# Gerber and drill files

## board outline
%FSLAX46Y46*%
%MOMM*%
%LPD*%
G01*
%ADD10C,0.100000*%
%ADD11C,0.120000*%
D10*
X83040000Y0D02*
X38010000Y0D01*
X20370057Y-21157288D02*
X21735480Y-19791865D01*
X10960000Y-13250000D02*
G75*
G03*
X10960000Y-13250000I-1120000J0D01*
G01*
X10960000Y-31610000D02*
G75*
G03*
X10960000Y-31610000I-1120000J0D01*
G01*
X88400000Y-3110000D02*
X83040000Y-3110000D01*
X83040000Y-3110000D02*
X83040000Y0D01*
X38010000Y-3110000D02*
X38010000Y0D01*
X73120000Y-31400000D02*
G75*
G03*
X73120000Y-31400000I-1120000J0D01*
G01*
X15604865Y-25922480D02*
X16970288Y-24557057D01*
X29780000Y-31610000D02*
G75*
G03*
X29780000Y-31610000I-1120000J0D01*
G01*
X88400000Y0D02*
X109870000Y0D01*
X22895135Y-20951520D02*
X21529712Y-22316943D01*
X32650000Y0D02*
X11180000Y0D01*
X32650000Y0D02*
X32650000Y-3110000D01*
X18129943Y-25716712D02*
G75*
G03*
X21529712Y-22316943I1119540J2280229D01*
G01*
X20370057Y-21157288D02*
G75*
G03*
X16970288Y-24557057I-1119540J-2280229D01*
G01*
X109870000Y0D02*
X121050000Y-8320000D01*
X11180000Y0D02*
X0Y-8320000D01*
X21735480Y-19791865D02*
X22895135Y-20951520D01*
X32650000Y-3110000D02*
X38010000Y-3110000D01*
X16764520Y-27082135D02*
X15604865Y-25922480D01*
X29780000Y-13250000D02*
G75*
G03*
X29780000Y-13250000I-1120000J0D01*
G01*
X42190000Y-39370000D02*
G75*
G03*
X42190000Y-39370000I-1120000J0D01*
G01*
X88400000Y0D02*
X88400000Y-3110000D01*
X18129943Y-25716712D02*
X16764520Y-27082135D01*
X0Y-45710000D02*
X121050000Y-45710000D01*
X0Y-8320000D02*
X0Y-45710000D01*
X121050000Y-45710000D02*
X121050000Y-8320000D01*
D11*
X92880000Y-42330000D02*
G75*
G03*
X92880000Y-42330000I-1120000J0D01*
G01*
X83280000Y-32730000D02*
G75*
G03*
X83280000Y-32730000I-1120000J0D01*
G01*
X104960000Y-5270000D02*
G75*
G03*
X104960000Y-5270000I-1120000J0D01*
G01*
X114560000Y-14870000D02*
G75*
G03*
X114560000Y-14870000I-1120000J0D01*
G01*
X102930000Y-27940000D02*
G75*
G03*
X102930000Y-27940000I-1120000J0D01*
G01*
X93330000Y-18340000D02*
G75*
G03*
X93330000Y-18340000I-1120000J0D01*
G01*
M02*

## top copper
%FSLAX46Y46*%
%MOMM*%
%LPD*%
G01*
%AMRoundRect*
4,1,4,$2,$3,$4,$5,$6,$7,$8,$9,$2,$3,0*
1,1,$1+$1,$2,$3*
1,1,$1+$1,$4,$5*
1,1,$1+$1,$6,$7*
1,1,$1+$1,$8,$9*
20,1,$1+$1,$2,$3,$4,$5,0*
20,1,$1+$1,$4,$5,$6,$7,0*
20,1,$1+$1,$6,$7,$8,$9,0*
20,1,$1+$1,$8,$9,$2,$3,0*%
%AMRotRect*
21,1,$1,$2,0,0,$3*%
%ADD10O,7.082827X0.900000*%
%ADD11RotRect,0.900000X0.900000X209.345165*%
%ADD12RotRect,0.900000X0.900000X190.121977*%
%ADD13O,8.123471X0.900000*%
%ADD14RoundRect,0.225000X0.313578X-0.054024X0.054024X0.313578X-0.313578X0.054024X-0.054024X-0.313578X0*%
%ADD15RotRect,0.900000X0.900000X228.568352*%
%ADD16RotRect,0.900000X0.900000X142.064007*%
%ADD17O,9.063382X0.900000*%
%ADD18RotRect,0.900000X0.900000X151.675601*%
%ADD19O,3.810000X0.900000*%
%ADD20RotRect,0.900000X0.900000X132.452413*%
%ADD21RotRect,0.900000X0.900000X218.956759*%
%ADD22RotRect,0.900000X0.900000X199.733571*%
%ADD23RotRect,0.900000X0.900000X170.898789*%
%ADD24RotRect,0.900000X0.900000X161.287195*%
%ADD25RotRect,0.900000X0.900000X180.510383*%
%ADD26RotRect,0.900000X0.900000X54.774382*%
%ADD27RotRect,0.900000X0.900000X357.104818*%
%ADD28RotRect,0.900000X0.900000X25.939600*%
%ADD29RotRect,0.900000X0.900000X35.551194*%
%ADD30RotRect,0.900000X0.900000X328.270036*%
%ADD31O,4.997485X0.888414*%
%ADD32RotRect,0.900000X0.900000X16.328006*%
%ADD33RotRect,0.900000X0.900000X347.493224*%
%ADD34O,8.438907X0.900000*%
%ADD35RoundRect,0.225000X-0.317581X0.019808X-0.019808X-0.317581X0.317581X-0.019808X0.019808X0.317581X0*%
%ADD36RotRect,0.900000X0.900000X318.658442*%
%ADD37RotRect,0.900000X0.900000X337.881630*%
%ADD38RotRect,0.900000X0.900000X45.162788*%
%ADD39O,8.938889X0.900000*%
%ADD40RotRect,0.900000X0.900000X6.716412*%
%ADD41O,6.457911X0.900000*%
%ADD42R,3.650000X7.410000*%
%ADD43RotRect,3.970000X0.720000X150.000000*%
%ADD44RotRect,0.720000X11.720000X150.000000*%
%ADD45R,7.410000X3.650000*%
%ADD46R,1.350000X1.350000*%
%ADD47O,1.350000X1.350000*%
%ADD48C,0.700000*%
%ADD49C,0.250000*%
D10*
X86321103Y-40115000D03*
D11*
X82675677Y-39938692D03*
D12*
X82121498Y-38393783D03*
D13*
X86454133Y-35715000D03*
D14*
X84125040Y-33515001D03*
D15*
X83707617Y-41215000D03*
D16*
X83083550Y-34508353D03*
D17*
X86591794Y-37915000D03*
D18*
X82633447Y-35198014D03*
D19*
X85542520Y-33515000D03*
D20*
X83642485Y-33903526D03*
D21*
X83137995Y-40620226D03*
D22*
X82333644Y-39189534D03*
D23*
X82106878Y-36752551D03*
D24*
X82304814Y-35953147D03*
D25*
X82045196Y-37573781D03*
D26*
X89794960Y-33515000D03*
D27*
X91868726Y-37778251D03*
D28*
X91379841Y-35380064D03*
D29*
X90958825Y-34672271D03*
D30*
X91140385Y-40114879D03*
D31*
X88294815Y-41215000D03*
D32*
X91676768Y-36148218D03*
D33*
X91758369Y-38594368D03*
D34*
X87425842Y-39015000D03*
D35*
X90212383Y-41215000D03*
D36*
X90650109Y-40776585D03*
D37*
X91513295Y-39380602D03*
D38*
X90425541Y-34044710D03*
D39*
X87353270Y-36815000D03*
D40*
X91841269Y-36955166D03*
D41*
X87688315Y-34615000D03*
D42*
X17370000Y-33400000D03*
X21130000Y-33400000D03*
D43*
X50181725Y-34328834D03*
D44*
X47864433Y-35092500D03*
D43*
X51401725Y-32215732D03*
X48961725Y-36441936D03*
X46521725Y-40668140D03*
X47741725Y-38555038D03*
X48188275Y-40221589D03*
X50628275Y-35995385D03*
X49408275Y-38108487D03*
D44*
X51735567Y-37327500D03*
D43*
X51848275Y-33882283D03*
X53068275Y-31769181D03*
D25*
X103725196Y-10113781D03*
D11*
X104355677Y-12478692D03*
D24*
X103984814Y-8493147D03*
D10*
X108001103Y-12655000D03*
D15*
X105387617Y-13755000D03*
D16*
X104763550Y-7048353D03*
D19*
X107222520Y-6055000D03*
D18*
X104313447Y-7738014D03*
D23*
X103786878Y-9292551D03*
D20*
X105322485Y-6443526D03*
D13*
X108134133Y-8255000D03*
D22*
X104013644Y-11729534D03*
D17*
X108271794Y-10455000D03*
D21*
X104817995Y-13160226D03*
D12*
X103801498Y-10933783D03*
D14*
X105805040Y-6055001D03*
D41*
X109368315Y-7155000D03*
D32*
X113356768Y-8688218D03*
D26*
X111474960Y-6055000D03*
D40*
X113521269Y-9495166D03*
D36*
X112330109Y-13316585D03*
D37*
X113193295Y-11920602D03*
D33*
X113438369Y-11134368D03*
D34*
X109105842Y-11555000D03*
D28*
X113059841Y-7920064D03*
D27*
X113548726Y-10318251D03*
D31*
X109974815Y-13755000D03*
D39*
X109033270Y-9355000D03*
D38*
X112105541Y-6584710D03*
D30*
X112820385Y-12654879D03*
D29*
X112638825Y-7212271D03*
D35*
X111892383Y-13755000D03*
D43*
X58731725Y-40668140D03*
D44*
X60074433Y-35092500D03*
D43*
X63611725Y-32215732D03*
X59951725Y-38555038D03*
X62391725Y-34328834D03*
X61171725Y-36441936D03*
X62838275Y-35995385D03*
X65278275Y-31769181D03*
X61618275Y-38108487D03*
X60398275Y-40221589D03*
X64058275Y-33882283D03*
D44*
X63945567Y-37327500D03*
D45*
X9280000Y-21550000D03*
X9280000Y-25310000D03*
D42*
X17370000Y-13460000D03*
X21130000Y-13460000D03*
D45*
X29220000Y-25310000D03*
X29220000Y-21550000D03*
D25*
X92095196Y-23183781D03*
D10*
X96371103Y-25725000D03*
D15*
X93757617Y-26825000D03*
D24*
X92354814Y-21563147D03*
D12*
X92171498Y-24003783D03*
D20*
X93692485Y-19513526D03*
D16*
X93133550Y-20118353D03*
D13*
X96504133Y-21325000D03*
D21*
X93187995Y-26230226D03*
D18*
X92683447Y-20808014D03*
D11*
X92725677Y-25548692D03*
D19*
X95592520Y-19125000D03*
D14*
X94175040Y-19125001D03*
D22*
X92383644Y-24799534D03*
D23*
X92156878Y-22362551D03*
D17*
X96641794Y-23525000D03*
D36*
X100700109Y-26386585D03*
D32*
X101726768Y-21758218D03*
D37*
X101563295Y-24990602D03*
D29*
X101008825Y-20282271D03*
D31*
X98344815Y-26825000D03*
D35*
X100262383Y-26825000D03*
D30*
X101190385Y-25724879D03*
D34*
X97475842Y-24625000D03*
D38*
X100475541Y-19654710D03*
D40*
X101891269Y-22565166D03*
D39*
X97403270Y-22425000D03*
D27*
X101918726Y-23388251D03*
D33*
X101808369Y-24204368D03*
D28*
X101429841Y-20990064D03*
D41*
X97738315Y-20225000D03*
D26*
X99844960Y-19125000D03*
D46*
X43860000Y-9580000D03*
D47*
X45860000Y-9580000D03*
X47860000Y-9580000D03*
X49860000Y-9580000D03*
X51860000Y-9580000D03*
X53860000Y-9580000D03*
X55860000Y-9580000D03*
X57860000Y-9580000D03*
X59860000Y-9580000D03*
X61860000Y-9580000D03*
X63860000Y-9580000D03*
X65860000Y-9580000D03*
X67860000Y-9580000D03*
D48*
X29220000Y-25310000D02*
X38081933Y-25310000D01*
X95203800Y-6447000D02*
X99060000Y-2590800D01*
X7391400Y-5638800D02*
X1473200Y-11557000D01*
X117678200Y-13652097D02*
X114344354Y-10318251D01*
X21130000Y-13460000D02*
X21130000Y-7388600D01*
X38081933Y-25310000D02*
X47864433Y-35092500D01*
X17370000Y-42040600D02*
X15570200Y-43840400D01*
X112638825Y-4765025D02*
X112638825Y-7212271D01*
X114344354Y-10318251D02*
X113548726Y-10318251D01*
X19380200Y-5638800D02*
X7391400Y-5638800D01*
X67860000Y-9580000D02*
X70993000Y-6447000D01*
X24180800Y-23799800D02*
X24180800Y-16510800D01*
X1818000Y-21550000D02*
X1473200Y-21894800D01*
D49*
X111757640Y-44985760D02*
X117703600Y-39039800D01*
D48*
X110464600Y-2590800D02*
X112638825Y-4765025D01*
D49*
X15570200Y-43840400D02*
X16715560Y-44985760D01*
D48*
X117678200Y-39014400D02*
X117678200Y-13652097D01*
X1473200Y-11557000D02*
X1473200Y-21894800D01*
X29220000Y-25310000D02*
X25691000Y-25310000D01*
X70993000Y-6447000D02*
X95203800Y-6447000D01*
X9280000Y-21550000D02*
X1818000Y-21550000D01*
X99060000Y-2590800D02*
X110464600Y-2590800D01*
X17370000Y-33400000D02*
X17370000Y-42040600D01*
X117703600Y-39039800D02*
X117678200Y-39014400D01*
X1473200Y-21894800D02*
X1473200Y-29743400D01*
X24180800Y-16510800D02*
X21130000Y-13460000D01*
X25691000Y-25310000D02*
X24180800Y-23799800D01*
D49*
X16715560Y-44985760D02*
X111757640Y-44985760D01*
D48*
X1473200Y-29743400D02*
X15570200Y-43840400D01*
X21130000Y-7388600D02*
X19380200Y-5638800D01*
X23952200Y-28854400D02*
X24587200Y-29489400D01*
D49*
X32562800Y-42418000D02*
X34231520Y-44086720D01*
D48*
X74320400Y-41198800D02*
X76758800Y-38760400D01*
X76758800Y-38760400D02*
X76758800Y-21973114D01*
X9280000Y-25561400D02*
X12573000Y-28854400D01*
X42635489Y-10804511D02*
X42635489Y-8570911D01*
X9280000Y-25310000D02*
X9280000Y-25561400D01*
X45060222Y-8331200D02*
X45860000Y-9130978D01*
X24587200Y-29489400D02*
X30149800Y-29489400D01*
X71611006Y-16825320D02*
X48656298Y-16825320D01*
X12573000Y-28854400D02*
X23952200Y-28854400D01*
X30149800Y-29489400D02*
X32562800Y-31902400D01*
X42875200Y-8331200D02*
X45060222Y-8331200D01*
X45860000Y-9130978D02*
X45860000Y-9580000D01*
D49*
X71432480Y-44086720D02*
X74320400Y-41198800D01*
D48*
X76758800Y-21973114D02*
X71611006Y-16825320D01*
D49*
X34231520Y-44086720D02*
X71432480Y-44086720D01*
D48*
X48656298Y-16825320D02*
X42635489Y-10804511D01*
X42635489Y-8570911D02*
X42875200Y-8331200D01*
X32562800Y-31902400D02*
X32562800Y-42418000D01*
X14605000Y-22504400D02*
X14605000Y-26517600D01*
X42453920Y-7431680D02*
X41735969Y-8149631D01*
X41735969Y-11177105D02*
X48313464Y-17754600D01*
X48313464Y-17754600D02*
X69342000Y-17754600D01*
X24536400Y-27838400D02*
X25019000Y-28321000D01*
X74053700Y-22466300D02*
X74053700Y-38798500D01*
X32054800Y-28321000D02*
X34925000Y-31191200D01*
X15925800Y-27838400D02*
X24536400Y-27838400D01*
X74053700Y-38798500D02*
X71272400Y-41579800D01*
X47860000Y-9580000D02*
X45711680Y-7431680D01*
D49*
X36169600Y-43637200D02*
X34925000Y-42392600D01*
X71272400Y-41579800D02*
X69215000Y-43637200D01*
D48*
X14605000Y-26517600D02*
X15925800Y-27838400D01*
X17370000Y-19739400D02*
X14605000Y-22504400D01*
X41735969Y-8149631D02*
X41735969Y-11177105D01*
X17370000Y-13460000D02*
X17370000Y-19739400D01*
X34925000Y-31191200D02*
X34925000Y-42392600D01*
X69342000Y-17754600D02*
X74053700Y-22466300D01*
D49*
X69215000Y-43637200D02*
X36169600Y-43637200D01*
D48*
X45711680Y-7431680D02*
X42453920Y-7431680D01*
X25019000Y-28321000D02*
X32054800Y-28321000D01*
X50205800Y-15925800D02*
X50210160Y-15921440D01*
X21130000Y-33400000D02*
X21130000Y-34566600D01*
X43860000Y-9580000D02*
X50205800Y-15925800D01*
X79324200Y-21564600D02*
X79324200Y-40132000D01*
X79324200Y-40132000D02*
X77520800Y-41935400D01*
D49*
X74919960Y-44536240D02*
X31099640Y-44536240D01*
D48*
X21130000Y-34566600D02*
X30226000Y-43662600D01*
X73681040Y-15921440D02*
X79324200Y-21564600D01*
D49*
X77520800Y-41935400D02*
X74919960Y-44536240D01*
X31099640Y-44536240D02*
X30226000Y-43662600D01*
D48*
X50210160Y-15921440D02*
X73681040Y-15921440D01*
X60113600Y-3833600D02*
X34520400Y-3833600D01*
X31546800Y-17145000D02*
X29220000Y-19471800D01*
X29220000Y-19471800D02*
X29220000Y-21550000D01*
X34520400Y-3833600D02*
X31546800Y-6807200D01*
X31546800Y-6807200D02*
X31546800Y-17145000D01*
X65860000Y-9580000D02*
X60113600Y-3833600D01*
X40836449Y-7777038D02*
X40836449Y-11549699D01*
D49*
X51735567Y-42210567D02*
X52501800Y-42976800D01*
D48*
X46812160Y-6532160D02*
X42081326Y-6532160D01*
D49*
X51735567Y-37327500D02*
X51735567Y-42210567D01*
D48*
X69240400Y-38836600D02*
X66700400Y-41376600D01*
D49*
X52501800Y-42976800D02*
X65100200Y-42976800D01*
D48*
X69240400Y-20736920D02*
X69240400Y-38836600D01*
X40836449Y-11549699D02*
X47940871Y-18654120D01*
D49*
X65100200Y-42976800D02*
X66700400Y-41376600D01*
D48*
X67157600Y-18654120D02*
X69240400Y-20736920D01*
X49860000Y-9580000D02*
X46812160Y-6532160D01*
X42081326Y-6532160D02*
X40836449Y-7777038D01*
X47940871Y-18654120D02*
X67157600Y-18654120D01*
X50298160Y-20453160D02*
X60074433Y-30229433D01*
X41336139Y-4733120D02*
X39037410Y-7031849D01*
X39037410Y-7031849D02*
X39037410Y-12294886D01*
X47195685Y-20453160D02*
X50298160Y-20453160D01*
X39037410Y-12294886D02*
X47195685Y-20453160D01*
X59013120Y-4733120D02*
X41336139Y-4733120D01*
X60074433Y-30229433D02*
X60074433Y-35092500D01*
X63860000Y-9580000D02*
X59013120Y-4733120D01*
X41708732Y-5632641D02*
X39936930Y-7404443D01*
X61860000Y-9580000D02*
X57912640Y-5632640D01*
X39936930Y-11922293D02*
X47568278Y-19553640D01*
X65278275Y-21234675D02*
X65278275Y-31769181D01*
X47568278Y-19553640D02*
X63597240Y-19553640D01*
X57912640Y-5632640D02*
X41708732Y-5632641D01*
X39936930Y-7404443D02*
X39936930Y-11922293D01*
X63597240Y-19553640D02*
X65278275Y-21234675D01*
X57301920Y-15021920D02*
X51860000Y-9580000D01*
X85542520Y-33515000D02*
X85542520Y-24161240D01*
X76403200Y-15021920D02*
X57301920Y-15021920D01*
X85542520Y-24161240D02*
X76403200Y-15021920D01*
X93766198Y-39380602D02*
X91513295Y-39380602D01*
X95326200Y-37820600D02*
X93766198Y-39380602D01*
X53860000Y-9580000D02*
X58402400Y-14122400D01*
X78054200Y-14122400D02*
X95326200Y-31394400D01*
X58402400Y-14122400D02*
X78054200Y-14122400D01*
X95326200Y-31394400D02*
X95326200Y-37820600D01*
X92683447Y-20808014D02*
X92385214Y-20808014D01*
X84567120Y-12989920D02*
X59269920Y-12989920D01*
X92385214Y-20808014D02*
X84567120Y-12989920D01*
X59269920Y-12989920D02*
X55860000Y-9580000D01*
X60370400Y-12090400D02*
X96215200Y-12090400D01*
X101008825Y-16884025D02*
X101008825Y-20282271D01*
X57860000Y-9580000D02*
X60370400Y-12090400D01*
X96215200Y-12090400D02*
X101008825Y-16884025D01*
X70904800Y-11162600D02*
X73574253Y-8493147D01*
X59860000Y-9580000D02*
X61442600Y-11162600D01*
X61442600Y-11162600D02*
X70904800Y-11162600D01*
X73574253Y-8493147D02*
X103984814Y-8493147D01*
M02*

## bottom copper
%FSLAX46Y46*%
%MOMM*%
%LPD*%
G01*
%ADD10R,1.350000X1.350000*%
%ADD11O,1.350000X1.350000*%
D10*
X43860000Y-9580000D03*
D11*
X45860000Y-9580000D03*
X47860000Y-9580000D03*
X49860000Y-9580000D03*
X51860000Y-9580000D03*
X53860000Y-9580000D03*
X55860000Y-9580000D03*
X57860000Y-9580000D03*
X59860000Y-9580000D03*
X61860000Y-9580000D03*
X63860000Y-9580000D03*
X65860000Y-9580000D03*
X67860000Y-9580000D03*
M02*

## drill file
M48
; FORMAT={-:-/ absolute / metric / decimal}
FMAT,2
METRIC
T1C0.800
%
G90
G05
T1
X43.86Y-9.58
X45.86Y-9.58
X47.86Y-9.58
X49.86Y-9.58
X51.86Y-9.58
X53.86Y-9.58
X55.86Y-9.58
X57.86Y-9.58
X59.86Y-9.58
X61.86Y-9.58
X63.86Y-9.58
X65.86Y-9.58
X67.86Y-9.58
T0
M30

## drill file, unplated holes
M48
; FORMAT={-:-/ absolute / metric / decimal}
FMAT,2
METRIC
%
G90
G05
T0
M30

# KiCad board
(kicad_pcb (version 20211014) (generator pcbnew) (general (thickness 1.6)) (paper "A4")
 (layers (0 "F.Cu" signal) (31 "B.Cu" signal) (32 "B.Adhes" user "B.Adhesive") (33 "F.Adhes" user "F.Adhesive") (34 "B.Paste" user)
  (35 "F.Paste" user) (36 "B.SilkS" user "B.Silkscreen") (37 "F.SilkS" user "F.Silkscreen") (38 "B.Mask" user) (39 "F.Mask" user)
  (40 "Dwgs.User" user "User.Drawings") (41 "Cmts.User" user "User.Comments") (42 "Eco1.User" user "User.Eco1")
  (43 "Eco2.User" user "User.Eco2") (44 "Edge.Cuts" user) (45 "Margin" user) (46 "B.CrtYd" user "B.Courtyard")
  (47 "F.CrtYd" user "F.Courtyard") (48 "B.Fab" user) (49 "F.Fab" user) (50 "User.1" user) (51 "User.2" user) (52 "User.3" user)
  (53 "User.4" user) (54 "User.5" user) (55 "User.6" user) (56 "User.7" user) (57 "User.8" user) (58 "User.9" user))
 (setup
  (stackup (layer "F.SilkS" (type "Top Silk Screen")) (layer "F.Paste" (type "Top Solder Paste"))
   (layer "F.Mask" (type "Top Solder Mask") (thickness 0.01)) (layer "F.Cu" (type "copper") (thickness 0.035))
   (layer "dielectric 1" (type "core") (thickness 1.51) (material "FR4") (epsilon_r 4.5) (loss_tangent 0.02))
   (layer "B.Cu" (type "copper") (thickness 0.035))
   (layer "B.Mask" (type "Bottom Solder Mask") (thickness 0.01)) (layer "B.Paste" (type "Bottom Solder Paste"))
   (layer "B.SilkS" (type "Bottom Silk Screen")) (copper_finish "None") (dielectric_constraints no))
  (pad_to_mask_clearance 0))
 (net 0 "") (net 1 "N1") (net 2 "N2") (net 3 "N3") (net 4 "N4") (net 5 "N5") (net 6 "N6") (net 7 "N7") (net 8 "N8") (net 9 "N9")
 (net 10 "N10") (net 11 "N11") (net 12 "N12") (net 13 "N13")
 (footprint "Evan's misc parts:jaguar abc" (layer "F.Cu") (at 86.96 37.53)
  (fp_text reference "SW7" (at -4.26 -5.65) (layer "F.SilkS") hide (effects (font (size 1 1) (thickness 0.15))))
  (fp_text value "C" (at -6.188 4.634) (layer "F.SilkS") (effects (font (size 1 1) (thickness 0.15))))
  (fp_circle (center 4.8 4.8) (end 5.92 4.8) (layer "Edge.Cuts") (width 0.12) (fill none))
  (fp_circle (center -4.8 -4.8) (end -3.68 -4.8) (layer "Edge.Cuts") (width 0.12) (fill none))
  (pad "1" smd oval (at -0.638897 2.585) (size 7.082827 0.9) (layers "F.Cu" "F.Mask") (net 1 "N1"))
  (pad "1" smd rect (at -4.284323 2.408692 209.3451645) (size 0.9 0.9) (layers "F.Cu" "F.Mask") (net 1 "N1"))
  (pad "1" smd rect (at -4.838502 0.863783 190.1219766) (size 0.9 0.9) (layers "F.Cu" "F.Mask") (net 1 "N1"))
  (pad "1" smd oval (at -0.505867 -1.815) (size 8.123471 0.9) (layers "F.Cu" "F.Mask") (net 1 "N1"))
  (pad "1" smd roundrect (at -2.83496 -4.014999 125.225) (size 0.9 0.9) (layers "F.Cu" "F.Mask") (roundrect_rratio 0.25) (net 1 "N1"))
  (pad "1" smd rect (at -3.252383 3.685 228.5683524) (size 0.9 0.9) (layers "F.Cu" "F.Mask") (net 1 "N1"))
  (pad "1" smd rect (at -3.87645 -3.021647 142.0640068) (size 0.9 0.9) (layers "F.Cu" "F.Mask") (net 1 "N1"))
  (pad "1" smd oval (at -0.368206 0.385) (size 9.063382 0.9) (layers "F.Cu" "F.Mask") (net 1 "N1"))
  (pad "1" smd rect (at -4.326553 -2.331986 151.6756008) (size 0.9 0.9) (layers "F.Cu" "F.Mask") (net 1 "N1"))
  (pad "1" smd oval (at -1.41748 -4.015) (size 3.81 0.9) (layers "F.Cu" "F.Mask") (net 1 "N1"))
  (pad "1" smd rect (at -3.317515 -3.626474 132.4524129) (size 0.9 0.9) (layers "F.Cu" "F.Mask") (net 1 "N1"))
  (pad "1" smd rect (at -3.822005 3.090226 218.9567585) (size 0.9 0.9) (layers "F.Cu" "F.Mask") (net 1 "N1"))
  (pad "1" smd rect (at -4.626356 1.659534 199.7335705) (size 0.9 0.9) (layers "F.Cu" "F.Mask") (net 1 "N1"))
  (pad "1" smd rect (at -4.853122 -0.777449 170.8987887) (size 0.9 0.9) (layers "F.Cu" "F.Mask") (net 1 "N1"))
  (pad "1" smd rect (at -4.655186 -1.576853 161.2871947) (size 0.9 0.9) (layers "F.Cu" "F.Mask") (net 1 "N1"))
  (pad "1" smd rect (at -4.914804 0.043781 180.5103826) (size 0.9 0.9) (layers "F.Cu" "F.Mask") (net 1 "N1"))
  (pad "2" smd rect (at 2.83496 -4.015 54.77438172) (size 0.9 0.9) (layers "F.Cu" "F.Mask") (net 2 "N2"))
  (pad "2" smd rect (at 4.908726 0.248251 357.104818) (size 0.9 0.9) (layers "F.Cu" "F.Mask") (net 2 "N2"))
  (pad "2" smd rect (at 4.419841 -2.149936 25.93959986) (size 0.9 0.9) (layers "F.Cu" "F.Mask") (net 2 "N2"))
  (pad "2" smd rect (at 3.998825 -2.857729 35.55119382) (size 0.9 0.9) (layers "F.Cu" "F.Mask") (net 2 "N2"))
  (pad "2" smd rect (at 4.180385 2.584879 328.2700361) (size 0.9 0.9) (layers "F.Cu" "F.Mask") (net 2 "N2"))
  (pad "2" smd oval (at 1.334815 3.685) (size 4.997485 0.888414) (layers "F.Cu" "F.Mask") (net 2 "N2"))
  (pad "2" smd rect (at 4.716768 -1.381782 16.32800591) (size 0.9 0.9) (layers "F.Cu" "F.Mask") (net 2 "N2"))
  (pad "2" smd rect (at 4.798369 1.064368 347.493224) (size 0.9 0.9) (layers "F.Cu" "F.Mask") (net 2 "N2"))
  (pad "2" smd oval (at 0.465842 1.485) (size 8.438907 0.9) (layers "F.Cu" "F.Mask") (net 2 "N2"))
  (pad "2" smd roundrect (at 3.252383 3.685 311.431) (size 0.9 0.9) (layers "F.Cu" "F.Mask") (roundrect_rratio 0.25) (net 2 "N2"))
  (pad "2" smd rect (at 3.690109 3.246585 318.6584422) (size 0.9 0.9) (layers "F.Cu" "F.Mask") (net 2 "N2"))
  (pad "2" smd rect (at 4.553295 1.850602 337.8816301) (size 0.9 0.9) (layers "F.Cu" "F.Mask") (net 2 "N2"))
  (pad "2" smd rect (at 3.465541 -3.48529 45.16278777) (size 0.9 0.9) (layers "F.Cu" "F.Mask") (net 2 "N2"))
  (pad "2" smd oval (at 0.39327 -0.715) (size 8.938889 0.9) (layers "F.Cu" "F.Mask") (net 2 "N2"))
  (pad "2" smd rect (at 4.881269 -0.574834 6.716411956) (size 0.9 0.9) (layers "F.Cu" "F.Mask") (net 2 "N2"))
  (pad "2" smd oval (at 0.728315 -2.915) (size 6.457911 0.9) (layers "F.Cu" "F.Mask") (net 2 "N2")))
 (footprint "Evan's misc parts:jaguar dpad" (layer "F.Cu") (at 19.25 33.4)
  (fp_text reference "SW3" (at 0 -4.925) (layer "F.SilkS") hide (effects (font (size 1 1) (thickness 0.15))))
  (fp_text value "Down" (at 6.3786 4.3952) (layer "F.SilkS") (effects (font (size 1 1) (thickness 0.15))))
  (pad "1" smd rect (at -1.88 0) (size 3.65 7.41) (layers "F.Cu" "F.Mask") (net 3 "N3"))
  (pad "2" smd rect (at 1.88 0) (size 3.65 7.41) (layers "F.Cu" "F.Mask") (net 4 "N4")))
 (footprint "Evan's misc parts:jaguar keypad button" (layer "F.Cu") (at 49.8 36.21 -30)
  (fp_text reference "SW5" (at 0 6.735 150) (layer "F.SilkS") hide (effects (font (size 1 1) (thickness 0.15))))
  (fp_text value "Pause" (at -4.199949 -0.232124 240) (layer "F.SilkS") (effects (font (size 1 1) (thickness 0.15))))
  (pad "1" smd rect (at -0.61 -1.82 150) (size 3.97 0.72) (layers "F.Cu" "F.Mask") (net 3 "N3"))
  (pad "1" smd rect (at -2.235 0 150) (size 0.72 11.72) (layers "F.Cu" "F.Mask") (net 3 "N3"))
  (pad "1" smd rect (at -0.61 -4.26 150) (size 3.97 0.72) (layers "F.Cu" "F.Mask") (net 3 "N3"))
  (pad "1" smd rect (at -0.61 0.62 150) (size 3.97 0.72) (layers "F.Cu" "F.Mask") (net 3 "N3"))
  (pad "1" smd rect (at -0.61 5.5 150) (size 3.97 0.72) (layers "F.Cu" "F.Mask") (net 3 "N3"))
  (pad "1" smd rect (at -0.61 3.06 150) (size 3.97 0.72) (layers "F.Cu" "F.Mask") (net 3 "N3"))
  (pad "2" smd rect (at 0.61 4.28 150) (size 3.97 0.72) (layers "F.Cu" "F.Mask") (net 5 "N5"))
  (pad "2" smd rect (at 0.61 -0.6 150) (size 3.97 0.72) (layers "F.Cu" "F.Mask") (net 5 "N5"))
  (pad "2" smd rect (at 0.61 1.84 150) (size 3.97 0.72) (layers "F.Cu" "F.Mask") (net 5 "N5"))
  (pad "2" smd rect (at 2.235 0 150) (size 0.72 11.72) (layers "F.Cu" "F.Mask") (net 5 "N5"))
  (pad "2" smd rect (at 0.61 -3.04 150) (size 3.97 0.72) (layers "F.Cu" "F.Mask") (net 5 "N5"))
  (pad "2" smd rect (at 0.61 -5.48 150) (size 3.97 0.72) (layers "F.Cu" "F.Mask") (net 5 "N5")))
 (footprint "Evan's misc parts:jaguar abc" (layer "F.Cu") (at 108.64 10.07)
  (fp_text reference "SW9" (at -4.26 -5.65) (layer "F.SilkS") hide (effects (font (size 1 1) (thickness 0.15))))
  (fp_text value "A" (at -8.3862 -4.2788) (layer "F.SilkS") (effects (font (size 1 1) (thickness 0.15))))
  (fp_circle (center -4.8 -4.8) (end -3.68 -4.8) (layer "Edge.Cuts") (width 0.12) (fill none))
  (fp_circle (center 4.8 4.8) (end 5.92 4.8) (layer "Edge.Cuts") (width 0.12) (fill none))
  (pad "1" smd rect (at -4.914804 0.043781 180.5103826) (size 0.9 0.9) (layers "F.Cu" "F.Mask") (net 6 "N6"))
  (pad "1" smd rect (at -4.284323 2.408692 209.3451645) (size 0.9 0.9) (layers "F.Cu" "F.Mask") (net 6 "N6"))
  (pad "1" smd rect (at -4.655186 -1.576853 161.2871947) (size 0.9 0.9) (layers "F.Cu" "F.Mask") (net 6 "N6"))
  (pad "1" smd oval (at -0.638897 2.585) (size 7.082827 0.9) (layers "F.Cu" "F.Mask") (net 6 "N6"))
  (pad "1" smd rect (at -3.252383 3.685 228.5683524) (size 0.9 0.9) (layers "F.Cu" "F.Mask") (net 6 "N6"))
  (pad "1" smd rect (at -3.87645 -3.021647 142.0640068) (size 0.9 0.9) (layers "F.Cu" "F.Mask") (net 6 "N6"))
  (pad "1" smd oval (at -1.41748 -4.015) (size 3.81 0.9) (layers "F.Cu" "F.Mask") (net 6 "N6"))
  (pad "1" smd rect (at -4.326553 -2.331986 151.6756008) (size 0.9 0.9) (layers "F.Cu" "F.Mask") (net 6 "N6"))
  (pad "1" smd rect (at -4.853122 -0.777449 170.8987887) (size 0.9 0.9) (layers "F.Cu" "F.Mask") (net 6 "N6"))
  (pad "1" smd rect (at -3.317515 -3.626474 132.4524129) (size 0.9 0.9) (layers "F.Cu" "F.Mask") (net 6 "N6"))
  (pad "1" smd oval (at -0.505867 -1.815) (size 8.123471 0.9) (layers "F.Cu" "F.Mask") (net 6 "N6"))
  (pad "1" smd rect (at -4.626356 1.659534 199.7335705) (size 0.9 0.9) (layers "F.Cu" "F.Mask") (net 6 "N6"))
  (pad "1" smd oval (at -0.368206 0.385) (size 9.063382 0.9) (layers "F.Cu" "F.Mask") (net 6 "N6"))
  (pad "1" smd rect (at -3.822005 3.090226 218.9567585) (size 0.9 0.9) (layers "F.Cu" "F.Mask") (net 6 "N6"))
  (pad "1" smd rect (at -4.838502 0.863783 190.1219766) (size 0.9 0.9) (layers "F.Cu" "F.Mask") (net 6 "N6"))
  (pad "1" smd roundrect (at -2.83496 -4.014999 125.225) (size 0.9 0.9) (layers "F.Cu" "F.Mask") (roundrect_rratio 0.25) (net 6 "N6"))
  (pad "2" smd oval (at 0.728315 -2.915) (size 6.457911 0.9) (layers "F.Cu" "F.Mask") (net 3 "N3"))
  (pad "2" smd rect (at 4.716768 -1.381782 16.32800591) (size 0.9 0.9) (layers "F.Cu" "F.Mask") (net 3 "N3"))
  (pad "2" smd rect (at 2.83496 -4.015 54.77438172) (size 0.9 0.9) (layers "F.Cu" "F.Mask") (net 3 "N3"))
  (pad "2" smd rect (at 4.881269 -0.574834 6.716411956) (size 0.9 0.9) (layers "F.Cu" "F.Mask") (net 3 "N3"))
  (pad "2" smd rect (at 3.690109 3.246585 318.6584422) (size 0.9 0.9) (layers "F.Cu" "F.Mask") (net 3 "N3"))
  (pad "2" smd rect (at 4.553295 1.850602 337.8816301) (size 0.9 0.9) (layers "F.Cu" "F.Mask") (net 3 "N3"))
  (pad "2" smd rect (at 4.798369 1.064368 347.493224) (size 0.9 0.9) (layers "F.Cu" "F.Mask") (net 3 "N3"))
  (pad "2" smd oval (at 0.465842 1.485) (size 8.438907 0.9) (layers "F.Cu" "F.Mask") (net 3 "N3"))
  (pad "2" smd rect (at 4.419841 -2.149936 25.93959986) (size 0.9 0.9) (layers "F.Cu" "F.Mask") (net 3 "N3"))
  (pad "2" smd rect (at 4.908726 0.248251 357.104818) (size 0.9 0.9) (layers "F.Cu" "F.Mask") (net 3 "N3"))
  (pad "2" smd oval (at 1.334815 3.685) (size 4.997485 0.888414) (layers "F.Cu" "F.Mask") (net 3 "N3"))
  (pad "2" smd oval (at 0.39327 -0.715) (size 8.938889 0.9) (layers "F.Cu" "F.Mask") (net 3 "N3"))
  (pad "2" smd rect (at 3.465541 -3.48529 45.16278777) (size 0.9 0.9) (layers "F.Cu" "F.Mask") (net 3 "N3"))
  (pad "2" smd rect (at 4.180385 2.584879 328.2700361) (size 0.9 0.9) (layers "F.Cu" "F.Mask") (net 3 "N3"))
  (pad "2" smd rect (at 3.998825 -2.857729 35.55119382) (size 0.9 0.9) (layers "F.Cu" "F.Mask") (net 3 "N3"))
  (pad "2" smd roundrect (at 3.252383 3.685 311.431) (size 0.9 0.9) (layers "F.Cu" "F.Mask") (roundrect_rratio 0.25) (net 3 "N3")))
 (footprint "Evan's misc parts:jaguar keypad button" (layer "F.Cu") (at 62.01 36.21 -30)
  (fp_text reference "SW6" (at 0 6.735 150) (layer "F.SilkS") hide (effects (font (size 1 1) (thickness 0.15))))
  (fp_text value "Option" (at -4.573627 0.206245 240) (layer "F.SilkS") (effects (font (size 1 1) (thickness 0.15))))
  (pad "1" smd rect (at -0.61 5.5 150) (size 3.97 0.72) (layers "F.Cu" "F.Mask") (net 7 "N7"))
  (pad "1" smd rect (at -2.235 0 150) (size 0.72 11.72) (layers "F.Cu" "F.Mask") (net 7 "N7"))
  (pad "1" smd rect (at -0.61 -4.26 150) (size 3.97 0.72) (layers "F.Cu" "F.Mask") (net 7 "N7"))
  (pad "1" smd rect (at -0.61 3.06 150) (size 3.97 0.72) (layers "F.Cu" "F.Mask") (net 7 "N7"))
  (pad "1" smd rect (at -0.61 -1.82 150) (size 3.97 0.72) (layers "F.Cu" "F.Mask") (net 7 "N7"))
  (pad "1" smd rect (at -0.61 0.62 150) (size 3.97 0.72) (layers "F.Cu" "F.Mask") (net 7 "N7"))
  (pad "2" smd rect (at 0.61 -0.6 150) (size 3.97 0.72) (layers "F.Cu" "F.Mask") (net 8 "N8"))
  (pad "2" smd rect (at 0.61 -5.48 150) (size 3.97 0.72) (layers "F.Cu" "F.Mask") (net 8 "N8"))
  (pad "2" smd rect (at 0.61 1.84 150) (size 3.97 0.72) (layers "F.Cu" "F.Mask") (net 8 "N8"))
  (pad "2" smd rect (at 0.61 4.28 150) (size 3.97 0.72) (layers "F.Cu" "F.Mask") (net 8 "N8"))
  (pad "2" smd rect (at 0.61 -3.04 150) (size 3.97 0.72) (layers "F.Cu" "F.Mask") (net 8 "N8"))
  (pad "2" smd rect (at 2.235 0 150) (size 0.72 11.72) (layers "F.Cu" "F.Mask") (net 8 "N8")))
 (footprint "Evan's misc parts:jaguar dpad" (layer "F.Cu") (at 9.28 23.43 -90)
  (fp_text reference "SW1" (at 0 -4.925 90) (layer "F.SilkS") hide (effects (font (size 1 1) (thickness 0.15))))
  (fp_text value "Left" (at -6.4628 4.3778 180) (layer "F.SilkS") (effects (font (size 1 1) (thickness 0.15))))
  (pad "1" smd rect (at -1.88 0 270) (size 3.65 7.41) (layers "F.Cu" "F.Mask") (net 3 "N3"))
  (pad "2" smd rect (at 1.88 0 270) (size 3.65 7.41) (layers "F.Cu" "F.Mask") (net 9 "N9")))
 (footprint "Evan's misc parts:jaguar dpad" (layer "F.Cu") (at 19.25 13.46)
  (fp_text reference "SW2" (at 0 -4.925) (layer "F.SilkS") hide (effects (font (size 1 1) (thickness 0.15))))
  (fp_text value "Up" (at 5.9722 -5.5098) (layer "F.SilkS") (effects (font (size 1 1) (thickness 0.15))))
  (pad "1" smd rect (at -1.88 0) (size 3.65 7.41) (layers "F.Cu" "F.Mask") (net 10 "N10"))
  (pad "2" smd rect (at 1.88 0) (size 3.65 7.41) (layers "F.Cu" "F.Mask") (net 3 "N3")))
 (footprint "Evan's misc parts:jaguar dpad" (layer "F.Cu") (at 29.22 23.43 90)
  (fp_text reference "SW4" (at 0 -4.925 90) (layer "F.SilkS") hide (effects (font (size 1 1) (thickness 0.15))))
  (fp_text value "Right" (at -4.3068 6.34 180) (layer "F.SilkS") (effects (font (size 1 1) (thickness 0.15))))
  (pad "1" smd rect (at -1.88 0 90) (size 3.65 7.41) (layers "F.Cu" "F.Mask") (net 3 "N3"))
  (pad "2" smd rect (at 1.88 0 90) (size 3.65 7.41) (layers "F.Cu" "F.Mask") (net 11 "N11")))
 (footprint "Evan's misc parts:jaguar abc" (layer "F.Cu") (at 97.01 23.14)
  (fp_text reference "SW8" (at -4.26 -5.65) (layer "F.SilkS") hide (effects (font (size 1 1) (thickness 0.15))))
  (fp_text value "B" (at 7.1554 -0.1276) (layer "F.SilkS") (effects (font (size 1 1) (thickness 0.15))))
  (fp_circle (center 4.8 4.8) (end 5.92 4.8) (layer "Edge.Cuts") (width 0.12) (fill none))
  (fp_circle (center -4.8 -4.8) (end -3.68 -4.8) (layer "Edge.Cuts") (width 0.12) (fill none))
  (pad "1" smd rect (at -4.914804 0.043781 180.5103826) (size 0.9 0.9) (layers "F.Cu" "F.Mask") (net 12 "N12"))
  (pad "1" smd oval (at -0.638897 2.585) (size 7.082827 0.9) (layers "F.Cu" "F.Mask") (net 12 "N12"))
  (pad "1" smd rect (at -3.252383 3.685 228.5683524) (size 0.9 0.9) (layers "F.Cu" "F.Mask") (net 12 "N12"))
  (pad "1" smd rect (at -4.655186 -1.576853 161.2871947) (size 0.9 0.9) (layers "F.Cu" "F.Mask") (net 12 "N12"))
  (pad "1" smd rect (at -4.838502 0.863783 190.1219766) (size 0.9 0.9) (layers "F.Cu" "F.Mask") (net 12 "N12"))
  (pad "1" smd rect (at -3.317515 -3.626474 132.4524129) (size 0.9 0.9) (layers "F.Cu" "F.Mask") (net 12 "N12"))
  (pad "1" smd rect (at -3.87645 -3.021647 142.0640068) (size 0.9 0.9) (layers "F.Cu" "F.Mask") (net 12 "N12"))
  (pad "1" smd oval (at -0.505867 -1.815) (size 8.123471 0.9) (layers "F.Cu" "F.Mask") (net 12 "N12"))
  (pad "1" smd rect (at -3.822005 3.090226 218.9567585) (size 0.9 0.9) (layers "F.Cu" "F.Mask") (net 12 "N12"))
  (pad "1" smd rect (at -4.326553 -2.331986 151.6756008) (size 0.9 0.9) (layers "F.Cu" "F.Mask") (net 12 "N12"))
  (pad "1" smd rect (at -4.284323 2.408692 209.3451645) (size 0.9 0.9) (layers "F.Cu" "F.Mask") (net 12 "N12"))
  (pad "1" smd oval (at -1.41748 -4.015) (size 3.81 0.9) (layers "F.Cu" "F.Mask") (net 12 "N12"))
  (pad "1" smd roundrect (at -2.83496 -4.014999 125.225) (size 0.9 0.9) (layers "F.Cu" "F.Mask") (roundrect_rratio 0.25) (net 12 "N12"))
  (pad "1" smd rect (at -4.626356 1.659534 199.7335705) (size 0.9 0.9) (layers "F.Cu" "F.Mask") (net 12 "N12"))
  (pad "1" smd rect (at -4.853122 -0.777449 170.8987887) (size 0.9 0.9) (layers "F.Cu" "F.Mask") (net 12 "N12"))
  (pad "1" smd oval (at -0.368206 0.385) (size 9.063382 0.9) (layers "F.Cu" "F.Mask") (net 12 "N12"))
  (pad "2" smd rect (at 3.690109 3.246585 318.6584422) (size 0.9 0.9) (layers "F.Cu" "F.Mask") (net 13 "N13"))
  (pad "2" smd rect (at 4.716768 -1.381782 16.32800591) (size 0.9 0.9) (layers "F.Cu" "F.Mask") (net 13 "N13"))
  (pad "2" smd rect (at 4.553295 1.850602 337.8816301) (size 0.9 0.9) (layers "F.Cu" "F.Mask") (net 13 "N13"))
  (pad "2" smd rect (at 3.998825 -2.857729 35.55119382) (size 0.9 0.9) (layers "F.Cu" "F.Mask") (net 13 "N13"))
  (pad "2" smd oval (at 1.334815 3.685) (size 4.997485 0.888414) (layers "F.Cu" "F.Mask") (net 13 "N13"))
  (pad "2" smd roundrect (at 3.252383 3.685 311.431) (size 0.9 0.9) (layers "F.Cu" "F.Mask") (roundrect_rratio 0.25) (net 13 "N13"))
  (pad "2" smd rect (at 4.180385 2.584879 328.2700361) (size 0.9 0.9) (layers "F.Cu" "F.Mask") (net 13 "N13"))
  (pad "2" smd oval (at 0.465842 1.485) (size 8.438907 0.9) (layers "F.Cu" "F.Mask") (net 13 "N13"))
  (pad "2" smd rect (at 3.465541 -3.48529 45.16278777) (size 0.9 0.9) (layers "F.Cu" "F.Mask") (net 13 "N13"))
  (pad "2" smd rect (at 4.881269 -0.574834 6.716411956) (size 0.9 0.9) (layers "F.Cu" "F.Mask") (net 13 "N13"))
  (pad "2" smd oval (at 0.39327 -0.715) (size 8.938889 0.9) (layers "F.Cu" "F.Mask") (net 13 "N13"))
  (pad "2" smd rect (at 4.908726 0.248251 357.104818) (size 0.9 0.9) (layers "F.Cu" "F.Mask") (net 13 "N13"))
  (pad "2" smd rect (at 4.798369 1.064368 347.493224) (size 0.9 0.9) (layers "F.Cu" "F.Mask") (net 13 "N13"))
  (pad "2" smd rect (at 4.419841 -2.149936 25.93959986) (size 0.9 0.9) (layers "F.Cu" "F.Mask") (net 13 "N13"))
  (pad "2" smd oval (at 0.728315 -2.915) (size 6.457911 0.9) (layers "F.Cu" "F.Mask") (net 13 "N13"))
  (pad "2" smd rect (at 2.83496 -4.015 54.77438172) (size 0.9 0.9) (layers "F.Cu" "F.Mask") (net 13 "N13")))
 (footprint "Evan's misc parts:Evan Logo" (layer "F.Cu") (at 45.3136 3.7084)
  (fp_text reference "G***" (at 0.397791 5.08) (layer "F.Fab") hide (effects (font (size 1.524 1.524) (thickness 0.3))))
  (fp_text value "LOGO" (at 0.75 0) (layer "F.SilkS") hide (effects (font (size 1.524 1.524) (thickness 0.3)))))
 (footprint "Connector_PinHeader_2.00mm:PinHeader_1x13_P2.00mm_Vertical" (layer "F.Cu") (at 43.86 9.58 90)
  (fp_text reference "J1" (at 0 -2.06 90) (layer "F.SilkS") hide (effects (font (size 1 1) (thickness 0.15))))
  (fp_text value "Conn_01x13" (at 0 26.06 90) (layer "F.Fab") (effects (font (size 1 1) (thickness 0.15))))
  (pad "1" thru_hole rect locked (at 0 0 90) (size 1.35 1.35) (drill 0.8) (layers *.Cu *.Mask) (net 4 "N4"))
  (pad "2" thru_hole oval locked (at 0 2 90) (size 1.35 1.35) (drill 0.8) (layers *.Cu *.Mask) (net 9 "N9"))
  (pad "3" thru_hole oval locked (at 0 4 90) (size 1.35 1.35) (drill 0.8) (layers *.Cu *.Mask) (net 10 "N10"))
  (pad "4" thru_hole oval locked (at 0 6 90) (size 1.35 1.35) (drill 0.8) (layers *.Cu *.Mask) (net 5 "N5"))
  (pad "5" thru_hole oval locked (at 0 8 90) (size 1.35 1.35) (drill 0.8) (layers *.Cu *.Mask) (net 1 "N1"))
  (pad "6" thru_hole oval locked (at 0 10 90) (size 1.35 1.35) (drill 0.8) (layers *.Cu *.Mask) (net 2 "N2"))
  (pad "7" thru_hole oval locked (at 0 12 90) (size 1.35 1.35) (drill 0.8) (layers *.Cu *.Mask) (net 12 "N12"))
  (pad "8" thru_hole oval locked (at 0 14 90) (size 1.35 1.35) (drill 0.8) (layers *.Cu *.Mask) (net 13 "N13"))
  (pad "9" thru_hole oval locked (at 0 16 90) (size 1.35 1.35) (drill 0.8) (layers *.Cu *.Mask) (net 6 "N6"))
  (pad "10" thru_hole oval locked (at 0 18 90) (size 1.35 1.35) (drill 0.8) (layers *.Cu *.Mask) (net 8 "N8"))
  (pad "11" thru_hole oval locked (at 0 20 90) (size 1.35 1.35) (drill 0.8) (layers *.Cu *.Mask) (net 7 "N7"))
  (pad "12" thru_hole oval locked (at 0 22 90) (size 1.35 1.35) (drill 0.8) (layers *.Cu *.Mask) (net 11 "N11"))
  (pad "13" thru_hole oval locked (at 0 24 90) (size 1.35 1.35) (drill 0.8) (layers *.Cu *.Mask) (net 3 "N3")))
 (gr_line (start 83.04 0) (end 38.01 0) (layer "Edge.Cuts") (width 0.1))
 (gr_line (start 20.370057 21.157288) (end 21.73548 19.791865) (layer "Edge.Cuts") (width 0.1))
 (gr_circle (center 9.84 13.25) (end 10.96 13.25) (layer "Edge.Cuts") (width 0.1) (fill none))
 (gr_circle (center 9.84 31.61) (end 10.96 31.61) (layer "Edge.Cuts") (width 0.1) (fill none))
 (gr_line (start 88.4 3.11) (end 83.04 3.11) (layer "Edge.Cuts") (width 0.1))
 (gr_line (start 83.04 3.11) (end 83.04 0) (layer "Edge.Cuts") (width 0.1))
 (gr_line (start 38.01 3.11) (end 38.01 0) (layer "Edge.Cuts") (width 0.1))
 (gr_circle (center 72 31.4) (end 73.12 31.4) (layer "Edge.Cuts") (width 0.1) (fill none))
 (gr_line (start 15.604865 25.92248) (end 16.970288 24.557057) (layer "Edge.Cuts") (width 0.1))
 (gr_circle (center 28.66 31.61) (end 29.78 31.61) (layer "Edge.Cuts") (width 0.1) (fill none))
 (gr_line (start 88.4 0) (end 109.87 0) (layer "Edge.Cuts") (width 0.1))
 (gr_line (start 22.895135 20.95152) (end 21.529712 22.316943) (layer "Edge.Cuts") (width 0.1))
 (gr_line (start 32.65 0) (end 11.18 0) (layer "Edge.Cuts") (width 0.1))
 (gr_line (start 32.65 0) (end 32.65 3.11) (layer "Edge.Cuts") (width 0.1))
 (gr_arc (start 21.529712 22.316943) (mid 21.045703 25.232703) (end 18.129943 25.716712) (layer "Edge.Cuts") (width 0.1))
 (gr_arc (start 16.970288 24.557057) (mid 17.454297 21.641297) (end 20.370057 21.157288) (layer "Edge.Cuts") (width 0.1))
 (gr_line (start 109.87 0) (end 121.05 8.32) (layer "Edge.Cuts") (width 0.1))
 (gr_line (start 11.18 0) (end 0 8.32) (layer "Edge.Cuts") (width 0.1))
 (gr_line (start 21.73548 19.791865) (end 22.895135 20.95152) (layer "Edge.Cuts") (width 0.1))
 (gr_line (start 32.65 3.11) (end 38.01 3.11) (layer "Edge.Cuts") (width 0.1))
 (gr_line (start 16.76452 27.082135) (end 15.604865 25.92248) (layer "Edge.Cuts") (width 0.1))
 (gr_circle (center 28.66 13.25) (end 29.78 13.25) (layer "Edge.Cuts") (width 0.1) (fill none))
 (gr_circle (center 41.07 39.37) (end 42.19 39.37) (layer "Edge.Cuts") (width 0.1) (fill none))
 (gr_line (start 88.4 0) (end 88.4 3.11) (layer "Edge.Cuts") (width 0.1))
 (gr_line (start 18.129943 25.716712) (end 16.76452 27.082135) (layer "Edge.Cuts") (width 0.1))
 (gr_line (start 0 45.71) (end 121.05 45.71) (layer "Edge.Cuts") (width 0.1))
 (gr_line (start 0 8.32) (end 0 45.71) (layer "Edge.Cuts") (width 0.1))
 (gr_line (start 121.05 45.71) (end 121.05 8.32) (layer "Edge.Cuts") (width 0.1))
 (segment (start 29.22 25.31) (end 38.081933 25.31) (width 0.7) (layer "F.Cu") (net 3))
 (segment (start 95.2038 6.447) (end 99.06 2.5908) (width 0.7) (layer "F.Cu") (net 3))
 (segment (start 7.3914 5.6388) (end 1.4732 11.557) (width 0.7) (layer "F.Cu") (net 3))
 (segment (start 117.6782 13.652097) (end 114.344354 10.318251) (width 0.7) (layer "F.Cu") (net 3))
 (segment (start 21.13 13.46) (end 21.13 7.3886) (width 0.7) (layer "F.Cu") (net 3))
 (segment (start 38.081933 25.31) (end 47.864433 35.0925) (width 0.7) (layer "F.Cu") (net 3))
 (segment (start 17.37 42.0406) (end 15.5702 43.8404) (width 0.7) (layer "F.Cu") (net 3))
 (segment (start 112.638825 4.765025) (end 112.638825 7.212271) (width 0.7) (layer "F.Cu") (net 3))
 (segment (start 114.344354 10.318251) (end 113.548726 10.318251) (width 0.7) (layer "F.Cu") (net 3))
 (segment (start 19.3802 5.6388) (end 7.3914 5.6388) (width 0.7) (layer "F.Cu") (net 3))
 (segment (start 67.86 9.58) (end 70.993 6.447) (width 0.7) (layer "F.Cu") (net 3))
 (segment (start 24.1808 23.7998) (end 24.1808 16.5108) (width 0.7) (layer "F.Cu") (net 3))
 (segment (start 1.818 21.55) (end 1.4732 21.8948) (width 0.7) (layer "F.Cu") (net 3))
 (segment (start 111.75764 44.98576) (end 117.7036 39.0398) (width 0.25) (layer "F.Cu") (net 3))
 (segment (start 110.4646 2.5908) (end 112.638825 4.765025) (width 0.7) (layer "F.Cu") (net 3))
 (segment (start 15.5702 43.8404) (end 16.71556 44.98576) (width 0.25) (layer "F.Cu") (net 3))
 (segment (start 117.6782 39.0144) (end 117.6782 13.652097) (width 0.7) (layer "F.Cu") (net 3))
 (segment (start 1.4732 11.557) (end 1.4732 21.8948) (width 0.7) (layer "F.Cu") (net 3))
 (segment (start 29.22 25.31) (end 25.691 25.31) (width 0.7) (layer "F.Cu") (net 3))
 (segment (start 70.993 6.447) (end 95.2038 6.447) (width 0.7) (layer "F.Cu") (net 3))
 (segment (start 9.28 21.55) (end 1.818 21.55) (width 0.7) (layer "F.Cu") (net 3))
 (segment (start 99.06 2.5908) (end 110.4646 2.5908) (width 0.7) (layer "F.Cu") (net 3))
 (segment (start 17.37 33.4) (end 17.37 42.0406) (width 0.7) (layer "F.Cu") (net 3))
 (segment (start 117.7036 39.0398) (end 117.6782 39.0144) (width 0.7) (layer "F.Cu") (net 3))
 (segment (start 1.4732 21.8948) (end 1.4732 29.7434) (width 0.7) (layer "F.Cu") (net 3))
 (segment (start 24.1808 16.5108) (end 21.13 13.46) (width 0.7) (layer "F.Cu") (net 3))
 (segment (start 25.691 25.31) (end 24.1808 23.7998) (width 0.7) (layer "F.Cu") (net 3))
 (segment (start 16.71556 44.98576) (end 111.75764 44.98576) (width 0.25) (layer "F.Cu") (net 3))
 (segment (start 1.4732 29.7434) (end 15.5702 43.8404) (width 0.7) (layer "F.Cu") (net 3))
 (segment (start 21.13 7.3886) (end 19.3802 5.6388) (width 0.7) (layer "F.Cu") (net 3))
 (segment (start 23.9522 28.8544) (end 24.5872 29.4894) (width 0.7) (layer "F.Cu") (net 9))
 (segment (start 32.5628 42.418) (end 34.23152 44.08672) (width 0.25) (layer "F.Cu") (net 9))
 (segment (start 74.3204 41.1988) (end 76.7588 38.7604) (width 0.7) (layer "F.Cu") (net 9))
 (segment (start 76.7588 38.7604) (end 76.7588 21.973114) (width 0.7) (layer "F.Cu") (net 9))
 (segment (start 9.28 25.5614) (end 12.573 28.8544) (width 0.7) (layer "F.Cu") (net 9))
 (segment (start 42.635489 10.804511) (end 42.635489 8.570911) (width 0.7) (layer "F.Cu") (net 9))
 (segment (start 9.28 25.31) (end 9.28 25.5614) (width 0.7) (layer "F.Cu") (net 9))
 (segment (start 45.060222 8.3312) (end 45.86 9.130978) (width 0.7) (layer "F.Cu") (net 9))
 (segment (start 24.5872 29.4894) (end 30.1498 29.4894) (width 0.7) (layer "F.Cu") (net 9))
 (segment (start 71.611006 16.82532) (end 48.656298 16.82532) (width 0.7) (layer "F.Cu") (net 9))
 (segment (start 12.573 28.8544) (end 23.9522 28.8544) (width 0.7) (layer "F.Cu") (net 9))
 (segment (start 30.1498 29.4894) (end 32.5628 31.9024) (width 0.7) (layer "F.Cu") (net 9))
 (segment (start 42.8752 8.3312) (end 45.060222 8.3312) (width 0.7) (layer "F.Cu") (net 9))
 (segment (start 45.86 9.130978) (end 45.86 9.58) (width 0.7) (layer "F.Cu") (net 9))
 (segment (start 71.43248 44.08672) (end 74.3204 41.1988) (width 0.25) (layer "F.Cu") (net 9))
 (segment (start 76.7588 21.973114) (end 71.611006 16.82532) (width 0.7) (layer "F.Cu") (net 9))
 (segment (start 34.23152 44.08672) (end 71.43248 44.08672) (width 0.25) (layer "F.Cu") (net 9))
 (segment (start 48.656298 16.82532) (end 42.635489 10.804511) (width 0.7) (layer "F.Cu") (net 9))
 (segment (start 42.635489 8.570911) (end 42.8752 8.3312) (width 0.7) (layer "F.Cu") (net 9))
 (segment (start 32.5628 31.9024) (end 32.5628 42.418) (width 0.7) (layer "F.Cu") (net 9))
 (segment (start 14.605 22.5044) (end 14.605 26.5176) (width 0.7) (layer "F.Cu") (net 10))
 (segment (start 42.45392 7.43168) (end 41.735969 8.149631) (width 0.7) (layer "F.Cu") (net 10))
 (segment (start 41.735969 11.177105) (end 48.313464 17.7546) (width 0.7) (layer "F.Cu") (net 10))
 (segment (start 48.313464 17.7546) (end 69.342 17.7546) (width 0.7) (layer "F.Cu") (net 10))
 (segment (start 24.5364 27.8384) (end 25.019 28.321) (width 0.7) (layer "F.Cu") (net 10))
 (segment (start 74.0537 22.4663) (end 74.0537 38.7985) (width 0.7) (layer "F.Cu") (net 10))
 (segment (start 32.0548 28.321) (end 34.925 31.1912) (width 0.7) (layer "F.Cu") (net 10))
 (segment (start 15.9258 27.8384) (end 24.5364 27.8384) (width 0.7) (layer "F.Cu") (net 10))
 (segment (start 74.0537 38.7985) (end 71.2724 41.5798) (width 0.7) (layer "F.Cu") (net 10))
 (segment (start 47.86 9.58) (end 45.71168 7.43168) (width 0.7) (layer "F.Cu") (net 10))
 (segment (start 36.1696 43.6372) (end 34.925 42.3926) (width 0.25) (layer "F.Cu") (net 10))
 (segment (start 71.2724 41.5798) (end 69.215 43.6372) (width 0.25) (layer "F.Cu") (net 10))
 (segment (start 14.605 26.5176) (end 15.9258 27.8384) (width 0.7) (layer "F.Cu") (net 10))
 (segment (start 17.37 19.7394) (end 14.605 22.5044) (width 0.7) (layer "F.Cu") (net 10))
 (segment (start 41.735969 8.149631) (end 41.735969 11.177105) (width 0.7) (layer "F.Cu") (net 10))
 (segment (start 17.37 13.46) (end 17.37 19.7394) (width 0.7) (layer "F.Cu") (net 10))
 (segment (start 34.925 31.1912) (end 34.925 42.3926) (width 0.7) (layer "F.Cu") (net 10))
 (segment (start 69.342 17.7546) (end 74.0537 22.4663) (width 0.7) (layer "F.Cu") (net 10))
 (segment (start 69.215 43.6372) (end 36.1696 43.6372) (width 0.25) (layer "F.Cu") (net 10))
 (segment (start 45.71168 7.43168) (end 42.45392 7.43168) (width 0.7) (layer "F.Cu") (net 10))
 (segment (start 25.019 28.321) (end 32.0548 28.321) (width 0.7) (layer "F.Cu") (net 10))
 (segment (start 50.2058 15.9258) (end 50.21016 15.92144) (width 0.7) (layer "F.Cu") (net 4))
 (segment (start 21.13 33.4) (end 21.13 34.5666) (width 0.7) (layer "F.Cu") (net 4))
 (segment (start 43.86 9.58) (end 50.2058 15.9258) (width 0.7) (layer "F.Cu") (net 4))
 (segment (start 79.3242 21.5646) (end 79.3242 40.132) (width 0.7) (layer "F.Cu") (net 4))
 (segment (start 79.3242 40.132) (end 77.5208 41.9354) (width 0.7) (layer "F.Cu") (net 4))
 (segment (start 74.91996 44.53624) (end 31.09964 44.53624) (width 0.25) (layer "F.Cu") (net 4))
 (segment (start 21.13 34.5666) (end 30.226 43.6626) (width 0.7) (layer "F.Cu") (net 4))
 (segment (start 73.68104 15.92144) (end 79.3242 21.5646) (width 0.7) (layer "F.Cu") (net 4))
 (segment (start 77.5208 41.9354) (end 74.91996 44.53624) (width 0.25) (layer "F.Cu") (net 4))
 (segment (start 31.09964 44.53624) (end 30.226 43.6626) (width 0.25) (layer "F.Cu") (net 4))
 (segment (start 50.21016 15.92144) (end 73.68104 15.92144) (width 0.7) (layer "F.Cu") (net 4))
 (segment (start 60.1136 3.8336) (end 34.5204 3.8336) (width 0.7) (layer "F.Cu") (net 11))
 (segment (start 31.5468 17.145) (end 29.22 19.4718) (width 0.7) (layer "F.Cu") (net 11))
 (segment (start 29.22 19.4718) (end 29.22 21.55) (width 0.7) (layer "F.Cu") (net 11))
 (segment (start 34.5204 3.8336) (end 31.5468 6.8072) (width 0.7) (layer "F.Cu") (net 11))
 (segment (start 31.5468 6.8072) (end 31.5468 17.145) (width 0.7) (layer "F.Cu") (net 11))
 (segment (start 65.86 9.58) (end 60.1136 3.8336) (width 0.7) (layer "F.Cu") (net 11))
 (segment (start 40.836449 7.777038) (end 40.836449 11.549699) (width 0.7) (layer "F.Cu") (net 5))
 (segment (start 51.735567 42.210567) (end 52.5018 42.9768) (width 0.25) (layer "F.Cu") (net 5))
 (segment (start 46.81216 6.53216) (end 42.081326 6.53216) (width 0.7) (layer "F.Cu") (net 5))
 (segment (start 51.735567 37.3275) (end 51.735567 42.210567) (width 0.25) (layer "F.Cu") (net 5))
 (segment (start 69.2404 38.8366) (end 66.7004 41.3766) (width 0.7) (layer "F.Cu") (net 5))
 (segment (start 52.5018 42.9768) (end 65.1002 42.9768) (width 0.25) (layer "F.Cu") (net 5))
 (segment (start 69.2404 20.73692) (end 69.2404 38.8366) (width 0.7) (layer "F.Cu") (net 5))
 (segment (start 40.836449 11.549699) (end 47.940871 18.65412) (width 0.7) (layer "F.Cu") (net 5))
 (segment (start 65.1002 42.9768) (end 66.7004 41.3766) (width 0.25) (layer "F.Cu") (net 5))
 (segment (start 67.1576 18.65412) (end 69.2404 20.73692) (width 0.7) (layer "F.Cu") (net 5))
 (segment (start 49.86 9.58) (end 46.81216 6.53216) (width 0.7) (layer "F.Cu") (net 5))
 (segment (start 42.081326 6.53216) (end 40.836449 7.777038) (width 0.7) (layer "F.Cu") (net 5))
 (segment (start 47.940871 18.65412) (end 67.1576 18.65412) (width 0.7) (layer "F.Cu") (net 5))
 (segment (start 50.29816 20.45316) (end 60.074433 30.229433) (width 0.7) (layer "F.Cu") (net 7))
 (segment (start 41.336139 4.73312) (end 39.03741 7.031849) (width 0.7) (layer "F.Cu") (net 7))
 (segment (start 39.03741 7.031849) (end 39.03741 12.294886) (width 0.7) (layer "F.Cu") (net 7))
 (segment (start 47.195685 20.45316) (end 50.29816 20.45316) (width 0.7) (layer "F.Cu") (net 7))
 (segment (start 39.03741 12.294886) (end 47.195685 20.45316) (width 0.7) (layer "F.Cu") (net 7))
 (segment (start 59.01312 4.73312) (end 41.336139 4.73312) (width 0.7) (layer "F.Cu") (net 7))
 (segment (start 60.074433 30.229433) (end 60.074433 35.0925) (width 0.7) (layer "F.Cu") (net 7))
 (segment (start 63.86 9.58) (end 59.01312 4.73312) (width 0.7) (layer "F.Cu") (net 7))
 (segment (start 41.708732 5.632641) (end 39.93693 7.404443) (width 0.7) (layer "F.Cu") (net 8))
 (segment (start 61.86 9.58) (end 57.91264 5.63264) (width 0.7) (layer "F.Cu") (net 8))
 (segment (start 39.93693 11.922293) (end 47.568278 19.55364) (width 0.7) (layer "F.Cu") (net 8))
 (segment (start 65.278275 21.234675) (end 65.278275 31.769181) (width 0.7) (layer "F.Cu") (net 8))
 (segment (start 47.568278 19.55364) (end 63.59724 19.55364) (width 0.7) (layer "F.Cu") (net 8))
 (segment (start 57.91264 5.63264) (end 41.708732 5.632641) (width 0.7) (layer "F.Cu") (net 8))
 (segment (start 39.93693 7.404443) (end 39.93693 11.922293) (width 0.7) (layer "F.Cu") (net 8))
 (segment (start 63.59724 19.55364) (end 65.278275 21.234675) (width 0.7) (layer "F.Cu") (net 8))
 (segment (start 57.30192 15.02192) (end 51.86 9.58) (width 0.7) (layer "F.Cu") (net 1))
 (segment (start 85.54252 33.515) (end 85.54252 24.16124) (width 0.7) (layer "F.Cu") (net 1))
 (segment (start 76.4032 15.02192) (end 57.30192 15.02192) (width 0.7) (layer "F.Cu") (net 1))
 (segment (start 85.54252 24.16124) (end 76.4032 15.02192) (width 0.7) (layer "F.Cu") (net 1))
 (segment (start 93.766198 39.380602) (end 91.513295 39.380602) (width 0.7) (layer "F.Cu") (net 2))
 (segment (start 95.3262 37.8206) (end 93.766198 39.380602) (width 0.7) (layer "F.Cu") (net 2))
 (segment (start 53.86 9.58) (end 58.4024 14.1224) (width 0.7) (layer "F.Cu") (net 2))
 (segment (start 78.0542 14.1224) (end 95.3262 31.3944) (width 0.7) (layer "F.Cu") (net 2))
 (segment (start 58.4024 14.1224) (end 78.0542 14.1224) (width 0.7) (layer "F.Cu") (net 2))
 (segment (start 95.3262 31.3944) (end 95.3262 37.8206) (width 0.7) (layer "F.Cu") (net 2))
 (segment (start 92.683447 20.808014) (end 92.385214 20.808014) (width 0.7) (layer "F.Cu") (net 12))
 (segment (start 84.56712 12.98992) (end 59.26992 12.98992) (width 0.7) (layer "F.Cu") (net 12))
 (segment (start 92.385214 20.808014) (end 84.56712 12.98992) (width 0.7) (layer "F.Cu") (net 12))
 (segment (start 59.26992 12.98992) (end 55.86 9.58) (width 0.7) (layer "F.Cu") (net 12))
 (segment (start 60.3704 12.0904) (end 96.2152 12.0904) (width 0.7) (layer "F.Cu") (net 13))
 (segment (start 101.008825 16.884025) (end 101.008825 20.282271) (width 0.7) (layer "F.Cu") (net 13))
 (segment (start 57.86 9.58) (end 60.3704 12.0904) (width 0.7) (layer "F.Cu") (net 13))
 (segment (start 96.2152 12.0904) (end 101.008825 16.884025) (width 0.7) (layer "F.Cu") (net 13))
 (segment (start 70.9048 11.1626) (end 73.574253 8.493147) (width 0.7) (layer "F.Cu") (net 6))
 (segment (start 59.86 9.58) (end 61.4426 11.1626) (width 0.7) (layer "F.Cu") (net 6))
 (segment (start 61.4426 11.1626) (end 70.9048 11.1626) (width 0.7) (layer "F.Cu") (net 6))
 (segment (start 73.574253 8.493147) (end 103.984814 8.493147) (width 0.7) (layer "F.Cu") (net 6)))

